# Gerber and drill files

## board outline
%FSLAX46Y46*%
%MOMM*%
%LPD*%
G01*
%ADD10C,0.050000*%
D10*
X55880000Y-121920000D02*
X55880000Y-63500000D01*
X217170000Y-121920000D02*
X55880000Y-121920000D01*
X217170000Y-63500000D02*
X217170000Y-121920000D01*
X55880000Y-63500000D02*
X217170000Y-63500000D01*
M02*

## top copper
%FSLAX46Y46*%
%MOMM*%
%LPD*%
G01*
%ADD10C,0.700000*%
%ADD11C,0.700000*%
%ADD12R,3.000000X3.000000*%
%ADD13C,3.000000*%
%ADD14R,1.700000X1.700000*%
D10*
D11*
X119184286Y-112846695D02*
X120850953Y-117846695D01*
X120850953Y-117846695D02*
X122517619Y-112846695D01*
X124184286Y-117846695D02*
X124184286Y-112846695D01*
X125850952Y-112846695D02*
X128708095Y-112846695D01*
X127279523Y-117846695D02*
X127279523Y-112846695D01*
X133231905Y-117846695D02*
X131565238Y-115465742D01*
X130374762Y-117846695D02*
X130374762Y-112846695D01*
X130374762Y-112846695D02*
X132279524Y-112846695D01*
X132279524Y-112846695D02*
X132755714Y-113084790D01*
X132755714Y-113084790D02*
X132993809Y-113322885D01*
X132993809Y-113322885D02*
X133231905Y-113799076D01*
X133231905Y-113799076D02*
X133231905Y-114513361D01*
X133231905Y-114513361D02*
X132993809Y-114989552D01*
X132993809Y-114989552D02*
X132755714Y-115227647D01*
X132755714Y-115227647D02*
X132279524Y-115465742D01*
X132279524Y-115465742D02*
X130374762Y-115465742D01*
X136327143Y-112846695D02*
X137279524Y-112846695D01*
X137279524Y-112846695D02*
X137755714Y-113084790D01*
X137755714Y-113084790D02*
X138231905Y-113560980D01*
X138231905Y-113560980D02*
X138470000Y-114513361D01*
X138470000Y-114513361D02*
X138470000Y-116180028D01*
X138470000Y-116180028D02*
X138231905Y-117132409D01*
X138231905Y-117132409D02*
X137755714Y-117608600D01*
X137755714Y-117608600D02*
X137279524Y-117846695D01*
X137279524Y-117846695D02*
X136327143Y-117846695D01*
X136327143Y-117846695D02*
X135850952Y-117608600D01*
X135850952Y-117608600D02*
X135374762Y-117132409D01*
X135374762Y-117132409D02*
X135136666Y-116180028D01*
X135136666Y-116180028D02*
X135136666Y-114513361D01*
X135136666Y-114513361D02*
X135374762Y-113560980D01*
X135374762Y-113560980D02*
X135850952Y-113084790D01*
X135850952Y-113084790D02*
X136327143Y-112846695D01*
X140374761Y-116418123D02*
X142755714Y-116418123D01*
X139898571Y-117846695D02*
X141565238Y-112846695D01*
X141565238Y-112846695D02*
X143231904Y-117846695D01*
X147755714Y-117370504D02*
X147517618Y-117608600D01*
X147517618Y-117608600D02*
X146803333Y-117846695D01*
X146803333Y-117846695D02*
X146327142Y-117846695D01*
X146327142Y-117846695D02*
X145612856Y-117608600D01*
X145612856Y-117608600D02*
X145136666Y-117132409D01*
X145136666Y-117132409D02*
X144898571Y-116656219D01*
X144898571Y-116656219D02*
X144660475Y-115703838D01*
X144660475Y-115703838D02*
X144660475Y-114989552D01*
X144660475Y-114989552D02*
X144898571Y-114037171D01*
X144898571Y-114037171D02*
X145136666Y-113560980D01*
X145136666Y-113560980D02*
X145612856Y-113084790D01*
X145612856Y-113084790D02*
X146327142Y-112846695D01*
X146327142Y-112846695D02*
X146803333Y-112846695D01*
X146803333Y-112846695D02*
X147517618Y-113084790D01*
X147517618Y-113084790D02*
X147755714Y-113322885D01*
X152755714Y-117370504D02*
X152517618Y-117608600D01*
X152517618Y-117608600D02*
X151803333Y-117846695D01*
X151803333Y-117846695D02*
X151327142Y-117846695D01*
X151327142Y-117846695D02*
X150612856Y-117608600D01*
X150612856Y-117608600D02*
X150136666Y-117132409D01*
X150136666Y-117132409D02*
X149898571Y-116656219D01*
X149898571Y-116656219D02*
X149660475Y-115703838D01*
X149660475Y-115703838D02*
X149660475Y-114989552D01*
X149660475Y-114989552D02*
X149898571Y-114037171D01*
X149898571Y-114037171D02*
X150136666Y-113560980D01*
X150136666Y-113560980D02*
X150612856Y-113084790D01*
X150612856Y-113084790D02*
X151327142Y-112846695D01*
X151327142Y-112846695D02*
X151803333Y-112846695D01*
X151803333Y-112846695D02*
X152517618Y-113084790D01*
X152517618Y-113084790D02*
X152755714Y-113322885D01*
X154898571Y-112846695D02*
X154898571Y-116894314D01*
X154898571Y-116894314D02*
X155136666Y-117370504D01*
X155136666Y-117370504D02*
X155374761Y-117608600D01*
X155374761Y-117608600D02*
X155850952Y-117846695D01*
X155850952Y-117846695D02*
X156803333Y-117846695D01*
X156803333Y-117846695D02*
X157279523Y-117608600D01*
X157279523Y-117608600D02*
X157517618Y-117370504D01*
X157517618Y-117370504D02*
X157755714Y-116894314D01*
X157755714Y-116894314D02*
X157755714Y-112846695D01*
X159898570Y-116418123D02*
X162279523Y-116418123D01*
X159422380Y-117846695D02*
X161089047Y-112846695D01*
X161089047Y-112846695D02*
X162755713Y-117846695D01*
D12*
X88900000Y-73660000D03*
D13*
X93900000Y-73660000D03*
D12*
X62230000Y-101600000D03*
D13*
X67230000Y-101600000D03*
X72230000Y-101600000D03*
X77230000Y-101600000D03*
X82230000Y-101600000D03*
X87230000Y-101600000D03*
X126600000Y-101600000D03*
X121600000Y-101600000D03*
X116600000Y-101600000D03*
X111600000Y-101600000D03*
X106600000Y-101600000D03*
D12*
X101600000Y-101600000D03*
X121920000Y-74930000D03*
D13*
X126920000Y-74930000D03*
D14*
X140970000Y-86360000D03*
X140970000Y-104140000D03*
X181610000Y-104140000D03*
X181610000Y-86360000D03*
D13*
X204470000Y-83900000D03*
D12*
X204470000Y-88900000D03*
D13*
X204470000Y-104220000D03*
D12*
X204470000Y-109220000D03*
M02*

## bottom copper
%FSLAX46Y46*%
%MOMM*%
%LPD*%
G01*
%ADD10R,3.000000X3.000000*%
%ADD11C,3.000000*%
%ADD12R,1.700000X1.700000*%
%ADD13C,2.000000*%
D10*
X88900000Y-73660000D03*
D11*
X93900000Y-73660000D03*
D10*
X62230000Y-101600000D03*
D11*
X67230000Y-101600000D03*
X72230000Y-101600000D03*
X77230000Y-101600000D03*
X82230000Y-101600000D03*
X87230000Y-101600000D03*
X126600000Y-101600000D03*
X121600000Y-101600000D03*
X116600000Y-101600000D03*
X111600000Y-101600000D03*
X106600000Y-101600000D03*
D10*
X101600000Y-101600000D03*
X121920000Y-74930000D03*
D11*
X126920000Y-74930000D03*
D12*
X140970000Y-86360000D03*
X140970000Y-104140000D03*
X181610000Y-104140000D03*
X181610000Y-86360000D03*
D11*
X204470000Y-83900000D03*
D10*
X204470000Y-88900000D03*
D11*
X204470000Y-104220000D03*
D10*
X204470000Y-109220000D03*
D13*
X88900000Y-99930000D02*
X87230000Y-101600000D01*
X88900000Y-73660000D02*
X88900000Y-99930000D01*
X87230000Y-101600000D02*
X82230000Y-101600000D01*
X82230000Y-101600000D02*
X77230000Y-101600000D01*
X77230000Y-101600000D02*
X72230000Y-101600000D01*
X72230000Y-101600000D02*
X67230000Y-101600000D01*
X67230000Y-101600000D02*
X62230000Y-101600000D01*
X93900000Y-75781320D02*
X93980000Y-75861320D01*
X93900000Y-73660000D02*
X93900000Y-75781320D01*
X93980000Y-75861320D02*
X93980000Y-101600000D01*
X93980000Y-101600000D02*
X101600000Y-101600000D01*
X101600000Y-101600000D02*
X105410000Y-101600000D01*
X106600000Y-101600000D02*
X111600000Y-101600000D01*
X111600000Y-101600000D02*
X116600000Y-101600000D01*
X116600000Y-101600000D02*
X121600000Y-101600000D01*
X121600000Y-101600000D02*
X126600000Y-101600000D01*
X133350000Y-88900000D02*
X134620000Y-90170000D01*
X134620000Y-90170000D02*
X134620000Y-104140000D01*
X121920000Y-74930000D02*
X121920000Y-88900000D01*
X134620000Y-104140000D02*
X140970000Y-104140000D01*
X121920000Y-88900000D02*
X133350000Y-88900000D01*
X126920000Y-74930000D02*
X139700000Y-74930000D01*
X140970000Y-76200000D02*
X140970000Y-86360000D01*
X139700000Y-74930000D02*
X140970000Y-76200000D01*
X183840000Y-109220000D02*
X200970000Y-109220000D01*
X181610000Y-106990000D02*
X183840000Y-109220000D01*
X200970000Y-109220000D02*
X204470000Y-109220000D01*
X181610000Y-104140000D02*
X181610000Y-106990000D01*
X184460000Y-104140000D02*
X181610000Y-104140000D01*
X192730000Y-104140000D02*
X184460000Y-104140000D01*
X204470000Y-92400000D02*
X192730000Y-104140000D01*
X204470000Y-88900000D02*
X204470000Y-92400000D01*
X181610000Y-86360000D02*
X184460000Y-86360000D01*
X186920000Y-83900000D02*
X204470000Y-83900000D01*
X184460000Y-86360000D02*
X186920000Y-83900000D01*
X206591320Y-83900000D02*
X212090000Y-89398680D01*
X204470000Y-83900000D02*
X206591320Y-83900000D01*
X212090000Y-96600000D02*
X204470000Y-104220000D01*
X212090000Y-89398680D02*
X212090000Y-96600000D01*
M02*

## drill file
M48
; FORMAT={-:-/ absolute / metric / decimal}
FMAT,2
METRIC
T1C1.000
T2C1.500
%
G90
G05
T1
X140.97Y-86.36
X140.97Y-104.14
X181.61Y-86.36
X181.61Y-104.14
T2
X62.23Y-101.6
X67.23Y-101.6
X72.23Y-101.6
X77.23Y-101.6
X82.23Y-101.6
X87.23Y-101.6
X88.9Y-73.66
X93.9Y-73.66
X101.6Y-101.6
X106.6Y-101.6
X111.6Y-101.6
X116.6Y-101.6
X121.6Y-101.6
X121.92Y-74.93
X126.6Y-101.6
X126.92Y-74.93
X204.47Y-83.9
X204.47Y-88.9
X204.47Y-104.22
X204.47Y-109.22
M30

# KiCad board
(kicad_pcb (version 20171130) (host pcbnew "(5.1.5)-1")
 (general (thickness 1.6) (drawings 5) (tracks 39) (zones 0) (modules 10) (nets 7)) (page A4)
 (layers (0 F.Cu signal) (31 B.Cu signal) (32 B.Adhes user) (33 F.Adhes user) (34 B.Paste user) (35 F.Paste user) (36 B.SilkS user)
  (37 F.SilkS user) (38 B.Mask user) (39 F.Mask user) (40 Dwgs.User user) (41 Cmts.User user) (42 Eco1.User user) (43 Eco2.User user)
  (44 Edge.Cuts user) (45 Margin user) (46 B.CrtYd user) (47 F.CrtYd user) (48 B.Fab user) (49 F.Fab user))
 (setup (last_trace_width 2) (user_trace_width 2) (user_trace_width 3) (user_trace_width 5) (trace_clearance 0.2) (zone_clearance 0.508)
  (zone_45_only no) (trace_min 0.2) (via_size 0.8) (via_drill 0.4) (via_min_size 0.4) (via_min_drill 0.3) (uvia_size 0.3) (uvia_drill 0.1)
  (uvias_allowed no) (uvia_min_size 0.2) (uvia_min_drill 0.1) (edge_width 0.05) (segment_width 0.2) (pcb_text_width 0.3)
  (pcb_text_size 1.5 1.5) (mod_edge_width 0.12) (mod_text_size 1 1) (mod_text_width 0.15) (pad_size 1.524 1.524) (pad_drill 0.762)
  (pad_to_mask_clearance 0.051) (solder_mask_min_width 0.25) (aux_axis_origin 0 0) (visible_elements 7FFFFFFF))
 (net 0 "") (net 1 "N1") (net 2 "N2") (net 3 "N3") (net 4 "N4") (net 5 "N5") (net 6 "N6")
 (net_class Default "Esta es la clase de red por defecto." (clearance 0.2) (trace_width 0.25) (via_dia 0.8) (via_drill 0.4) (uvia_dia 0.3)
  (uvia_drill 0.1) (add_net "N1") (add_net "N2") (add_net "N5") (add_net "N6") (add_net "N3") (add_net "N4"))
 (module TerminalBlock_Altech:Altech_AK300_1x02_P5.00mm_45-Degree (layer F.Cu) (at 88.9 73.66)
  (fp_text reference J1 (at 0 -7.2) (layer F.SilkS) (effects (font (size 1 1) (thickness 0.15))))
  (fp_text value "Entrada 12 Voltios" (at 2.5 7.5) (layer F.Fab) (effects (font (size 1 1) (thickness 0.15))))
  (pad 1 thru_hole rect (at 0 0) (size 3 3) (drill 1.5) (layers *.Cu *.Mask) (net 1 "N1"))
  (pad 2 thru_hole circle (at 5 0) (size 3 3) (drill 1.5) (layers *.Cu *.Mask) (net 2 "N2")))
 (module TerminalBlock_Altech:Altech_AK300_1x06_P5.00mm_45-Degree (layer F.Cu) (at 62.23 101.6)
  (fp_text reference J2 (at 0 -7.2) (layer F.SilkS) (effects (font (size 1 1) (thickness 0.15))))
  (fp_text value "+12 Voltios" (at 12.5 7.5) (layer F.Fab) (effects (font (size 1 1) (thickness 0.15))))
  (pad 1 thru_hole rect (at 0 0) (size 3 3) (drill 1.5) (layers *.Cu *.Mask) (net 1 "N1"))
  (pad 2 thru_hole circle (at 5 0) (size 3 3) (drill 1.5) (layers *.Cu *.Mask) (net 1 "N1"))
  (pad 3 thru_hole circle (at 10 0) (size 3 3) (drill 1.5) (layers *.Cu *.Mask) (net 1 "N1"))
  (pad 4 thru_hole circle (at 15 0) (size 3 3) (drill 1.5) (layers *.Cu *.Mask) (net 1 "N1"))
  (pad 5 thru_hole circle (at 20 0) (size 3 3) (drill 1.5) (layers *.Cu *.Mask) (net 1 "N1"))
  (pad 6 thru_hole circle (at 25 0) (size 3 3) (drill 1.5) (layers *.Cu *.Mask) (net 1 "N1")))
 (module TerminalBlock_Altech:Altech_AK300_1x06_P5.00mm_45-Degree (layer F.Cu) (at 101.6 101.6)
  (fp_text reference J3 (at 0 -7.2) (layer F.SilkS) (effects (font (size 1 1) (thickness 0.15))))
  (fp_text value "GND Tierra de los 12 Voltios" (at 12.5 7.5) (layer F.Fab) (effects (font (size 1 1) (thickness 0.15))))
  (pad 6 thru_hole circle (at 25 0) (size 3 3) (drill 1.5) (layers *.Cu *.Mask) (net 2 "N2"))
  (pad 5 thru_hole circle (at 20 0) (size 3 3) (drill 1.5) (layers *.Cu *.Mask) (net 2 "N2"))
  (pad 4 thru_hole circle (at 15 0) (size 3 3) (drill 1.5) (layers *.Cu *.Mask) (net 2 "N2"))
  (pad 3 thru_hole circle (at 10 0) (size 3 3) (drill 1.5) (layers *.Cu *.Mask) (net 2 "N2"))
  (pad 2 thru_hole circle (at 5 0) (size 3 3) (drill 1.5) (layers *.Cu *.Mask) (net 2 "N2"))
  (pad 1 thru_hole rect (at 0 0) (size 3 3) (drill 1.5) (layers *.Cu *.Mask) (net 2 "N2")))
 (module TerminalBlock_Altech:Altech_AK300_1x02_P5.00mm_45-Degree (layer F.Cu) (at 121.92 74.93)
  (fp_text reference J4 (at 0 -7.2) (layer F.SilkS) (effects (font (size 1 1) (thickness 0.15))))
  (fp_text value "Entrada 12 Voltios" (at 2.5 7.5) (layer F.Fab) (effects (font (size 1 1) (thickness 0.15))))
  (pad 1 thru_hole rect (at 0 0) (size 3 3) (drill 1.5) (layers *.Cu *.Mask) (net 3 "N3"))
  (pad 2 thru_hole circle (at 5 0) (size 3 3) (drill 1.5) (layers *.Cu *.Mask) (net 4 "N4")))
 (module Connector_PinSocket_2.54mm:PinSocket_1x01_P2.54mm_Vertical (layer F.Cu) (at 140.97 86.36)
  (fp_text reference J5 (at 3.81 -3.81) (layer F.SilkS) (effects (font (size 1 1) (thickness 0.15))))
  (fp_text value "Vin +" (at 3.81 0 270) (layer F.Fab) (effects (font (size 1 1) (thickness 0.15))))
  (pad 1 thru_hole rect (at 0 0) (size 1.7 1.7) (drill 1) (layers *.Cu *.Mask) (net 4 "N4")))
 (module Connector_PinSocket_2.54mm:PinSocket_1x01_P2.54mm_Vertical (layer F.Cu) (at 140.97 104.14)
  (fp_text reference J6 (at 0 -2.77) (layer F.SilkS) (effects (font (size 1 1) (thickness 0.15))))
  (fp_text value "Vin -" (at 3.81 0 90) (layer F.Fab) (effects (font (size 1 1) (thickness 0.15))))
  (pad 1 thru_hole rect (at 0 0) (size 1.7 1.7) (drill 1) (layers *.Cu *.Mask) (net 3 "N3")))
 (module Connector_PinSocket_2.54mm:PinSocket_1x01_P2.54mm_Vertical (layer F.Cu) (at 181.61 104.14)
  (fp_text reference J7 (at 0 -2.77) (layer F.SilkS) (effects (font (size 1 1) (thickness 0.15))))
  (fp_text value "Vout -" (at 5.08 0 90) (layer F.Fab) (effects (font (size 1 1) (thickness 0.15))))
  (pad 1 thru_hole rect (at 0 0) (size 1.7 1.7) (drill 1) (layers *.Cu *.Mask) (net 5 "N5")))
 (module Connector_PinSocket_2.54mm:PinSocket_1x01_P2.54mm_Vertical (layer F.Cu) (at 181.61 86.36)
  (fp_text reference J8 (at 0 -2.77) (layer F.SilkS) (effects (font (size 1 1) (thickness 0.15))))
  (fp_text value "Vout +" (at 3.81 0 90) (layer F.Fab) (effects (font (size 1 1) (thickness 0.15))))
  (pad 1 thru_hole rect (at 0 0) (size 1.7 1.7) (drill 1) (layers *.Cu *.Mask) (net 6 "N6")))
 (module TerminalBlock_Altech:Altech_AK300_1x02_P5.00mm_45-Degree (layer F.Cu) (at 204.47 88.9 90)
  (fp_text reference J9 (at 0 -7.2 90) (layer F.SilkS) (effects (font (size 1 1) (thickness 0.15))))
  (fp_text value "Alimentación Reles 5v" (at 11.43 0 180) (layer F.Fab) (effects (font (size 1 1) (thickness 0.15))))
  (pad 2 thru_hole circle (at 5 0 90) (size 3 3) (drill 1.5) (layers *.Cu *.Mask) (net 6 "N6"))
  (pad 1 thru_hole rect (at 0 0 90) (size 3 3) (drill 1.5) (layers *.Cu *.Mask) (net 5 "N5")))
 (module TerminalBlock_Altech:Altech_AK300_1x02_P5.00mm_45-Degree (layer F.Cu) (at 204.47 109.22 90)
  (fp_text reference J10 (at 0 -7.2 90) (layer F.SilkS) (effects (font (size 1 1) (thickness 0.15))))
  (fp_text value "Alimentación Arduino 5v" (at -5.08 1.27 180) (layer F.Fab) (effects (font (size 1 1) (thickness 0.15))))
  (pad 2 thru_hole circle (at 5 0 90) (size 3 3) (drill 1.5) (layers *.Cu *.Mask) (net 6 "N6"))
  (pad 1 thru_hole rect (at 0 0 90) (size 3 3) (drill 1.5) (layers *.Cu *.Mask) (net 5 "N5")))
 (gr_line (start 55.88 121.92) (end 55.88 63.5) (layer Edge.Cuts) (width 0.05))
 (gr_line (start 217.17 121.92) (end 55.88 121.92) (layer Edge.Cuts) (width 0.05))
 (gr_line (start 217.17 63.5) (end 217.17 121.92) (layer Edge.Cuts) (width 0.05))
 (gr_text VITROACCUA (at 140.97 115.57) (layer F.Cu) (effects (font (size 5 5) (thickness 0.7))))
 (gr_line (start 55.88 63.5) (end 217.17 63.5) (layer Edge.Cuts) (width 0.05))
 (segment (start 88.9 99.93) (end 87.23 101.6) (width 2) (layer B.Cu) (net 1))
 (segment (start 88.9 73.66) (end 88.9 99.93) (width 2) (layer B.Cu) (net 1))
 (segment (start 87.23 101.6) (end 82.23 101.6) (width 2) (layer B.Cu) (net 1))
 (segment (start 82.23 101.6) (end 77.23 101.6) (width 2) (layer B.Cu) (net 1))
 (segment (start 77.23 101.6) (end 72.23 101.6) (width 2) (layer B.Cu) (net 1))
 (segment (start 72.23 101.6) (end 67.23 101.6) (width 2) (layer B.Cu) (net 1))
 (segment (start 67.23 101.6) (end 62.23 101.6) (width 2) (layer B.Cu) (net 1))
 (segment (start 93.9 75.78132) (end 93.98 75.86132) (width 2) (layer B.Cu) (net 2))
 (segment (start 93.9 73.66) (end 93.9 75.78132) (width 2) (layer B.Cu) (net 2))
 (segment (start 93.98 75.86132) (end 93.98 101.6) (width 2) (layer B.Cu) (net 2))
 (segment (start 93.98 101.6) (end 101.6 101.6) (width 2) (layer B.Cu) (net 2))
 (segment (start 101.6 101.6) (end 105.41 101.6) (width 2) (layer B.Cu) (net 2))
 (segment (start 106.6 101.6) (end 111.6 101.6) (width 2) (layer B.Cu) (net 2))
 (segment (start 111.6 101.6) (end 116.6 101.6) (width 2) (layer B.Cu) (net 2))
 (segment (start 116.6 101.6) (end 121.6 101.6) (width 2) (layer B.Cu) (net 2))
 (segment (start 121.6 101.6) (end 126.6 101.6) (width 2) (layer B.Cu) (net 2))
 (segment (start 133.35 88.9) (end 134.62 90.17) (width 2) (layer B.Cu) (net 3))
 (segment (start 134.62 90.17) (end 134.62 104.14) (width 2) (layer B.Cu) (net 3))
 (segment (start 121.92 74.93) (end 121.92 88.9) (width 2) (layer B.Cu) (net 3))
 (segment (start 134.62 104.14) (end 140.97 104.14) (width 2) (layer B.Cu) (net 3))
 (segment (start 121.92 88.9) (end 133.35 88.9) (width 2) (layer B.Cu) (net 3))
 (segment (start 126.92 74.93) (end 139.7 74.93) (width 2) (layer B.Cu) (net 4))
 (segment (start 140.97 76.2) (end 140.97 86.36) (width 2) (layer B.Cu) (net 4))
 (segment (start 139.7 74.93) (end 140.97 76.2) (width 2) (layer B.Cu) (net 4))
 (segment (start 183.84 109.22) (end 200.97 109.22) (width 2) (layer B.Cu) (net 5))
 (segment (start 181.61 106.99) (end 183.84 109.22) (width 2) (layer B.Cu) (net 5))
 (segment (start 200.97 109.22) (end 204.47 109.22) (width 2) (layer B.Cu) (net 5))
 (segment (start 181.61 104.14) (end 181.61 106.99) (width 2) (layer B.Cu) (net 5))
 (segment (start 184.46 104.14) (end 181.61 104.14) (width 2) (layer B.Cu) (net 5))
 (segment (start 192.73 104.14) (end 184.46 104.14) (width 2) (layer B.Cu) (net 5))
 (segment (start 204.47 92.4) (end 192.73 104.14) (width 2) (layer B.Cu) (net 5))
 (segment (start 204.47 88.9) (end 204.47 92.4) (width 2) (layer B.Cu) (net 5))
 (segment (start 181.61 86.36) (end 184.46 86.36) (width 2) (layer B.Cu) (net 6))
 (segment (start 186.92 83.9) (end 204.47 83.9) (width 2) (layer B.Cu) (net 6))
 (segment (start 184.46 86.36) (end 186.92 83.9) (width 2) (layer B.Cu) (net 6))
 (segment (start 206.59132 83.9) (end 212.09 89.39868) (width 2) (layer B.Cu) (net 6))
 (segment (start 204.47 83.9) (end 206.59132 83.9) (width 2) (layer B.Cu) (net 6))
 (segment (start 212.09 96.6) (end 204.47 104.22) (width 2) (layer B.Cu) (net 6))
 (segment (start 212.09 89.39868) (end 212.09 96.6) (width 2) (layer B.Cu) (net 6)))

